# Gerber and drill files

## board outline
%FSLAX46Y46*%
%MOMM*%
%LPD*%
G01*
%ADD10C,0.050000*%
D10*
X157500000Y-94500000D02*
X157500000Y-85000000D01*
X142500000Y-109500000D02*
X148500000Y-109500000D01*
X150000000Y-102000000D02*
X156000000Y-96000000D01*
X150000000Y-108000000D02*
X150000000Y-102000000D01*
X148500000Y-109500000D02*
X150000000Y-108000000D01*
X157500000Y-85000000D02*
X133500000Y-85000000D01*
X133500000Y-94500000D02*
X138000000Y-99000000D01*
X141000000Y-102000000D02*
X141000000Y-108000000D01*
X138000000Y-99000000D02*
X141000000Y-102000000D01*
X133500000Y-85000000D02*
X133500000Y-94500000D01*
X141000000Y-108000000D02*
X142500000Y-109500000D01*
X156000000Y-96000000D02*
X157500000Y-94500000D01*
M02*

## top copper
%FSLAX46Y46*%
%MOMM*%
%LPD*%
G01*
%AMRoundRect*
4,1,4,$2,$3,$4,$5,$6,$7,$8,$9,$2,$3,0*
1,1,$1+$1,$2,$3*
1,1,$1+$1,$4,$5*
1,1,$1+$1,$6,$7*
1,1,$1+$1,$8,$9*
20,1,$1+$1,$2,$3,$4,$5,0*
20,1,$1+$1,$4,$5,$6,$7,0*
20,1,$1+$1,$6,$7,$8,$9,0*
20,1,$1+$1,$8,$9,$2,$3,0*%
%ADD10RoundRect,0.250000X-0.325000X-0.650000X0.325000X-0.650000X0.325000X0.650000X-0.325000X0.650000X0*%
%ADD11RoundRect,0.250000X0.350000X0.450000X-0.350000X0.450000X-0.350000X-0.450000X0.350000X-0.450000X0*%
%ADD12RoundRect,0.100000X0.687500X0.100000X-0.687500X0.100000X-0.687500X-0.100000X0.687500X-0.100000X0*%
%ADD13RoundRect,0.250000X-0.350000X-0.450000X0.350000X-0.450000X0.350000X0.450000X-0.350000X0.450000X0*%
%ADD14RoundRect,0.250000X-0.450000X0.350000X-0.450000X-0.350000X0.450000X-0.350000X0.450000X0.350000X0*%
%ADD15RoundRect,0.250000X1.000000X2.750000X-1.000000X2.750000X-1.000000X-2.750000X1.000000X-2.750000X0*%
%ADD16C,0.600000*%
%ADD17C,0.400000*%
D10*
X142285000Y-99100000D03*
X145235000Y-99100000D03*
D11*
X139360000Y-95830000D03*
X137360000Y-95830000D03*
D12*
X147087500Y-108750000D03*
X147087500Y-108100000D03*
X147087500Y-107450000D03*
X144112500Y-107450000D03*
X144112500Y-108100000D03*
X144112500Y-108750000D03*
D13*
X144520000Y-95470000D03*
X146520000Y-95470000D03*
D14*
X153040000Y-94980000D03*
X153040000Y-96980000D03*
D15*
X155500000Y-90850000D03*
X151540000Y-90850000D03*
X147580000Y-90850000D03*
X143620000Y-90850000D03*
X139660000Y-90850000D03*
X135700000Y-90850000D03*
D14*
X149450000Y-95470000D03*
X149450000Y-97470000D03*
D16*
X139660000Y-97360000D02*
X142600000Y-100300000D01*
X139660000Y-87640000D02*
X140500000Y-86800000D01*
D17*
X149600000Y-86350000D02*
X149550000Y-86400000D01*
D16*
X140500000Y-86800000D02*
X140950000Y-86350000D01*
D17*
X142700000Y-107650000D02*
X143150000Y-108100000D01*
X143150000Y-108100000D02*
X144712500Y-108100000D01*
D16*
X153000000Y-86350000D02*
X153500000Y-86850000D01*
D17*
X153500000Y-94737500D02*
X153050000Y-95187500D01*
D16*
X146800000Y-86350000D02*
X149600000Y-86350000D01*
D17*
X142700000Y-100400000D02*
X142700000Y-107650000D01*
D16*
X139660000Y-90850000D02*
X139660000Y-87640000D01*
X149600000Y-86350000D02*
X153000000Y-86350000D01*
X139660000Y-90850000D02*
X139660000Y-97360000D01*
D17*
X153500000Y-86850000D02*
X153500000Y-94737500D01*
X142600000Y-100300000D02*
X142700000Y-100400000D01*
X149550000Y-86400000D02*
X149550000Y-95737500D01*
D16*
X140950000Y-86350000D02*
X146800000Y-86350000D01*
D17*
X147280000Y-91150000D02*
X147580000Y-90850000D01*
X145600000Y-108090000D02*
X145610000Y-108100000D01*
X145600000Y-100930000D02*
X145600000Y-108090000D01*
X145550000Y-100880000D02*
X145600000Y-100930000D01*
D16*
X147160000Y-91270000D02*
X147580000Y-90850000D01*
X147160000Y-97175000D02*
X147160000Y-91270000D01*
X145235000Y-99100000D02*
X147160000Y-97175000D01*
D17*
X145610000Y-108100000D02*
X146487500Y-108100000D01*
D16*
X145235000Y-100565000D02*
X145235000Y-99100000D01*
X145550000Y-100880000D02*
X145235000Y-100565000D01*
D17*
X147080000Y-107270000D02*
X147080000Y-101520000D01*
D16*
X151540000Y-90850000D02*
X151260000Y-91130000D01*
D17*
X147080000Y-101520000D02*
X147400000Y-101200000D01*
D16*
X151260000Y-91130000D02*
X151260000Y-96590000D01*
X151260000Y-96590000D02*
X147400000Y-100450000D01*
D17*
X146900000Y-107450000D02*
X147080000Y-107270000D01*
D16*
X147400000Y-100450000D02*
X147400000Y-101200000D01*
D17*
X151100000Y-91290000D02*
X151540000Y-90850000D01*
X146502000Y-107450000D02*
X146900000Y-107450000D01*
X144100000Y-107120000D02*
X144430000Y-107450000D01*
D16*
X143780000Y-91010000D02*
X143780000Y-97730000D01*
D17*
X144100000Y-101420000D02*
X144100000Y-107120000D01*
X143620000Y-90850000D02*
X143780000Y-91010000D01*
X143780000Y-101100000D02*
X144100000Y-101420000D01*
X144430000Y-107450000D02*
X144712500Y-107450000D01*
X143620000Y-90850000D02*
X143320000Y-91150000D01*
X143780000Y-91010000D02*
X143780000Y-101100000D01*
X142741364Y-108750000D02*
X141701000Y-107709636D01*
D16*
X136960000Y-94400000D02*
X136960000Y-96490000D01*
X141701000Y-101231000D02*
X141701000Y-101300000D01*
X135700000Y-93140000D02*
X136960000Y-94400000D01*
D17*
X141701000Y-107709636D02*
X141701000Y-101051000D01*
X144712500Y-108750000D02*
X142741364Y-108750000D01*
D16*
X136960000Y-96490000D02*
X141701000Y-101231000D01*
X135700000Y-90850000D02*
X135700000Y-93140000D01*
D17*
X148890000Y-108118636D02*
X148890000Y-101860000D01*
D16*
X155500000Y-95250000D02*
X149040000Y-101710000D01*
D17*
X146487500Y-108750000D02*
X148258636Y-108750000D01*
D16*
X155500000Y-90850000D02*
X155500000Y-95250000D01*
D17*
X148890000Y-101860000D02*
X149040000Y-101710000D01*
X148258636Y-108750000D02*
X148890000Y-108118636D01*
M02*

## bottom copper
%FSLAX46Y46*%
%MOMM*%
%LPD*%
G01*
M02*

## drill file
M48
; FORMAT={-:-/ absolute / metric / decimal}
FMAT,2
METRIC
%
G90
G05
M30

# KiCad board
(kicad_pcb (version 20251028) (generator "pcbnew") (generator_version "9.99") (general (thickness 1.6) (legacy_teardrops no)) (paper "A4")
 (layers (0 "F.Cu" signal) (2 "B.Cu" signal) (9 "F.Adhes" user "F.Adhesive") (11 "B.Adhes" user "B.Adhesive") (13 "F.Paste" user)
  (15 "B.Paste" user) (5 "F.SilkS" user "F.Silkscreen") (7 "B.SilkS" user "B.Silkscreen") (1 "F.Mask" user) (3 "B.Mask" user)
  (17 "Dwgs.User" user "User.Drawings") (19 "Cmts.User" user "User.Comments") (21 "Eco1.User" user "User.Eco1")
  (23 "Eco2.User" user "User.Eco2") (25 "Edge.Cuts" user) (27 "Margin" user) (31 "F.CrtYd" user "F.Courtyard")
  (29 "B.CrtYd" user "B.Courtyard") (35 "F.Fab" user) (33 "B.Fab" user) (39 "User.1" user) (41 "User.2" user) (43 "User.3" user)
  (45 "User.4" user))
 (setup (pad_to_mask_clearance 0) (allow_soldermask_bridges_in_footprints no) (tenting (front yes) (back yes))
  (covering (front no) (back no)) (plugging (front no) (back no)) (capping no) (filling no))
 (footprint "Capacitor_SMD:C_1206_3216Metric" (layer "F.Cu") (at 143.76 99.1)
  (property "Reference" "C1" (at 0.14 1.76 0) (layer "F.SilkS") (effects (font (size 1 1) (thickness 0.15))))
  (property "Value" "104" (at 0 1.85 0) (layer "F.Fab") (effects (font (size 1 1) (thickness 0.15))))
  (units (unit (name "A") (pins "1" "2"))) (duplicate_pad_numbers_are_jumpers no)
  (pad "1" smd roundrect (at -1.475 0) (size 1.15 1.8) (layers "F.Cu" "F.Mask" "F.Paste") (roundrect_rratio 0.217391) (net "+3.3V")
   (tenting (front none) (back none)))
  (pad "2" smd roundrect (at 1.475 0) (size 1.15 1.8) (layers "F.Cu" "F.Mask" "F.Paste") (roundrect_rratio 0.217391) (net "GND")
   (tenting (front none) (back none))))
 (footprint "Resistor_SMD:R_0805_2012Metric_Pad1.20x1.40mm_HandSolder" (layer "F.Cu") (at 138.36 95.83 180)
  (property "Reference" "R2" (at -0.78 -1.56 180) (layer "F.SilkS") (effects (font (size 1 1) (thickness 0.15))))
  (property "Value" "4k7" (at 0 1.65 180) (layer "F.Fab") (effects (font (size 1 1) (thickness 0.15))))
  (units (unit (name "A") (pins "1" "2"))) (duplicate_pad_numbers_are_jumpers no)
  (pad "1" smd roundrect (at -1 0 180) (size 1.2 1.4) (layers "F.Cu" "F.Mask" "F.Paste") (roundrect_rratio 0.208333) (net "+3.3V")
   (tenting (front none) (back none)))
  (pad "2" smd roundrect (at 1 0 180) (size 1.2 1.4) (layers "F.Cu" "F.Mask" "F.Paste") (roundrect_rratio 0.208333) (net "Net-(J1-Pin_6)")
   (tenting (front none) (back none))))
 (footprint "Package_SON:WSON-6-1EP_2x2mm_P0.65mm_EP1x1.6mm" (layer "F.Cu") (at 145.6 108.1 180)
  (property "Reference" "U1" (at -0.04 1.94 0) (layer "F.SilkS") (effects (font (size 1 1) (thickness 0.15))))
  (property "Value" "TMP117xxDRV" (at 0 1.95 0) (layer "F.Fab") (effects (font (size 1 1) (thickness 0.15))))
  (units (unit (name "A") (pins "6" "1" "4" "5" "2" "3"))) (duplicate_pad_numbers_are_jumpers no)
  (pad "1" smd roundrect (at -0.8875 -0.65 180) (size 1.575 0.4) (drill (offset -0.6 0)) (layers "F.Cu" "F.Mask" "F.Paste")
   (roundrect_rratio 0.25) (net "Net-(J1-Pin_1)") (tenting (front none) (back none)))
  (pad "2" smd roundrect (at -0.8875 0 180) (size 1.575 0.4) (drill (offset -0.6 0)) (layers "F.Cu" "F.Mask" "F.Paste")
   (roundrect_rratio 0.25) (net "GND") (tenting (front none) (back none)))
  (pad "3" smd roundrect (at -0.8875 0.65 180) (size 1.575 0.4) (drill (offset -0.6 0)) (layers "F.Cu" "F.Mask" "F.Paste")
   (roundrect_rratio 0.25) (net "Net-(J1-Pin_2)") (tenting (front none) (back none)))
  (pad "4" smd roundrect (at 0.8875 0.65 180) (size 1.575 0.4) (drill (offset 0.6 0)) (layers "F.Cu" "F.Mask" "F.Paste")
   (roundrect_rratio 0.25) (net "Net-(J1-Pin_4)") (tenting (front none) (back none)))
  (pad "5" smd roundrect (at 0.8875 0 180) (size 1.575 0.4) (drill (offset 0.6 0)) (layers "F.Cu" "F.Mask" "F.Paste")
   (roundrect_rratio 0.25) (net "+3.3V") (tenting (front none) (back none)))
  (pad "6" smd roundrect (at 0.8875 -0.65 180) (size 1.575 0.4) (drill (offset 0.6 0)) (layers "F.Cu" "F.Mask" "F.Paste")
   (roundrect_rratio 0.25) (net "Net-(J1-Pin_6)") (tenting (front none) (back none))))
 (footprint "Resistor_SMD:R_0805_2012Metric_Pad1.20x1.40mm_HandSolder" (layer "F.Cu") (at 145.52 95.47)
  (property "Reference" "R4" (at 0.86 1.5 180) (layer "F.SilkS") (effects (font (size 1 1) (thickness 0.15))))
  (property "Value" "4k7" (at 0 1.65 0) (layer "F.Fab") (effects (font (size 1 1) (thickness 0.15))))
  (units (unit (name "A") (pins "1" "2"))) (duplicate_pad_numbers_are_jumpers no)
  (pad "1" smd roundrect (at -1 0) (size 1.2 1.4) (layers "F.Cu" "F.Mask" "F.Paste") (roundrect_rratio 0.208333) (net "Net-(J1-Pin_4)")
   (tenting (front none) (back none)))
  (pad "2" smd roundrect (at 1 0) (size 1.2 1.4) (layers "F.Cu" "F.Mask" "F.Paste") (roundrect_rratio 0.208333) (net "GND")
   (tenting (front none) (back none))))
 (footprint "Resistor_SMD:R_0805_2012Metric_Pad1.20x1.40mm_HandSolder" (layer "F.Cu") (at 153.04 95.98 -90)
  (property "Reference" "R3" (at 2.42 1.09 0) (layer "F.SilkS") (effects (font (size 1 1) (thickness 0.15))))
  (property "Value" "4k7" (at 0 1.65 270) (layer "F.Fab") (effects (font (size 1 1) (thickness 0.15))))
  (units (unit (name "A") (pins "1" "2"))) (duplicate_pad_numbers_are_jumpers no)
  (pad "1" smd roundrect (at -1 0 270) (size 1.2 1.4) (layers "F.Cu" "F.Mask" "F.Paste") (roundrect_rratio 0.208333) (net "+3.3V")
   (tenting (front none) (back none)))
  (pad "2" smd roundrect (at 1 0 270) (size 1.2 1.4) (layers "F.Cu" "F.Mask" "F.Paste") (roundrect_rratio 0.208333) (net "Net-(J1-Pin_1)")
   (tenting (front none) (back none))))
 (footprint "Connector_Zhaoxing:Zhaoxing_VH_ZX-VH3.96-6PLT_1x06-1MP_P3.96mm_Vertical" (layer "F.Cu") (at 145.6 88.85 180)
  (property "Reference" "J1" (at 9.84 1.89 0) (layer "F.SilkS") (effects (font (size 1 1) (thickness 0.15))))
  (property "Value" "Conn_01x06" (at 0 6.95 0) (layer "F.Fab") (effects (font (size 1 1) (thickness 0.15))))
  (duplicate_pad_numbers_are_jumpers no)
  (pad "1" smd roundrect (at -9.9 -2 180) (size 2.5 6) (layers "F.Cu" "F.Mask" "F.Paste") (roundrect_rratio 0.1) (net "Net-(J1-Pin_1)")
   (tenting (front none) (back none)))
  (pad "2" smd roundrect (at -5.94 -2 180) (size 2.5 6) (layers "F.Cu" "F.Mask" "F.Paste") (roundrect_rratio 0.1) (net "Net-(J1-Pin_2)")
   (tenting (front none) (back none)))
  (pad "3" smd roundrect (at -1.98 -2 180) (size 2.5 6) (layers "F.Cu" "F.Mask" "F.Paste") (roundrect_rratio 0.1) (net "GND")
   (tenting (front none) (back none)))
  (pad "4" smd roundrect (at 1.98 -2 180) (size 2.5 6) (layers "F.Cu" "F.Mask" "F.Paste") (roundrect_rratio 0.1) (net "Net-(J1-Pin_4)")
   (tenting (front none) (back none)))
  (pad "5" smd roundrect (at 5.94 -2 180) (size 2.5 6) (layers "F.Cu" "F.Mask" "F.Paste") (roundrect_rratio 0.1) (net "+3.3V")
   (tenting (front none) (back none)))
  (pad "6" smd roundrect (at 9.9 -2 180) (size 2.5 6) (layers "F.Cu" "F.Mask" "F.Paste") (roundrect_rratio 0.1) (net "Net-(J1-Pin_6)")
   (tenting (front none) (back none))))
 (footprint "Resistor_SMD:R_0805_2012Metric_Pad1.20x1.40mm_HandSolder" (layer "F.Cu") (at 149.45 96.47 -90)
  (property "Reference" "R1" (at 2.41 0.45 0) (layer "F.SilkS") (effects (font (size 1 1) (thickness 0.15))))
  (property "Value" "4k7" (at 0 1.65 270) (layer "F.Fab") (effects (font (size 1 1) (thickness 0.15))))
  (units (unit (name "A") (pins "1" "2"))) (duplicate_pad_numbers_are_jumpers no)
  (pad "1" smd roundrect (at -1 0 270) (size 1.2 1.4) (layers "F.Cu" "F.Mask" "F.Paste") (roundrect_rratio 0.208333) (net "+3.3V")
   (tenting (front none) (back none)))
  (pad "2" smd roundrect (at 1 0 270) (size 1.2 1.4) (layers "F.Cu" "F.Mask" "F.Paste") (roundrect_rratio 0.208333) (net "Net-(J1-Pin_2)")
   (tenting (front none) (back none))))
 (gr_line (start 157.5 94.5) (end 157.5 85) (stroke (width 0.05) (type default)) (layer "Edge.Cuts"))
 (gr_line (start 142.5 109.5) (end 148.5 109.5) (stroke (width 0.05) (type default)) (layer "Edge.Cuts"))
 (gr_line (start 150 102) (end 156 96) (stroke (width 0.05) (type default)) (layer "Edge.Cuts"))
 (gr_line (start 150 108) (end 150 102) (stroke (width 0.05) (type default)) (layer "Edge.Cuts"))
 (gr_line (start 148.5 109.5) (end 150 108) (stroke (width 0.05) (type default)) (layer "Edge.Cuts"))
 (gr_line (start 157.5 85) (end 133.5 85) (stroke (width 0.05) (type default)) (layer "Edge.Cuts"))
 (gr_line (start 133.5 94.5) (end 138 99) (stroke (width 0.05) (type default)) (layer "Edge.Cuts"))
 (gr_line (start 141 102) (end 141 108) (stroke (width 0.05) (type default)) (layer "Edge.Cuts"))
 (gr_line (start 138 99) (end 141 102) (stroke (width 0.05) (type default)) (layer "Edge.Cuts"))
 (gr_line (start 133.5 85) (end 133.5 94.5) (stroke (width 0.05) (type default)) (layer "Edge.Cuts"))
 (gr_line (start 141 108) (end 142.5 109.5) (stroke (width 0.05) (type default)) (layer "Edge.Cuts"))
 (gr_line (start 156 96) (end 157.5 94.5) (stroke (width 0.05) (type default)) (layer "Edge.Cuts"))
 (segment (start 139.66 97.36) (end 142.6 100.3) (width 0.6) (layer "F.Cu") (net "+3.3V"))
 (segment (start 139.66 87.64) (end 140.5 86.8) (width 0.6) (layer "F.Cu") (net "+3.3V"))
 (segment (start 149.6 86.35) (end 149.55 86.4) (width 0.4) (layer "F.Cu") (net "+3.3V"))
 (segment (start 140.5 86.8) (end 140.95 86.35) (width 0.6) (layer "F.Cu") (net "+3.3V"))
 (segment (start 142.7 107.65) (end 143.15 108.1) (width 0.4) (layer "F.Cu") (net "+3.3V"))
 (segment (start 143.15 108.1) (end 144.7125 108.1) (width 0.4) (layer "F.Cu") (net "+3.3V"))
 (segment (start 153 86.35) (end 153.5 86.85) (width 0.6) (layer "F.Cu") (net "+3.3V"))
 (segment (start 153.5 94.7375) (end 153.05 95.1875) (width 0.4) (layer "F.Cu") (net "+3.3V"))
 (segment (start 146.8 86.35) (end 149.6 86.35) (width 0.6) (layer "F.Cu") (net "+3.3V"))
 (segment (start 142.7 100.4) (end 142.7 107.65) (width 0.4) (layer "F.Cu") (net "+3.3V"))
 (segment (start 139.66 90.85) (end 139.66 87.64) (width 0.6) (layer "F.Cu") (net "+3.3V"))
 (segment (start 149.6 86.35) (end 153 86.35) (width 0.6) (layer "F.Cu") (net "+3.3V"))
 (segment (start 139.66 90.85) (end 139.66 97.36) (width 0.6) (layer "F.Cu") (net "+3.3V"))
 (segment (start 153.5 86.85) (end 153.5 94.7375) (width 0.4) (layer "F.Cu") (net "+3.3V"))
 (segment (start 142.6 100.3) (end 142.7 100.4) (width 0.4) (layer "F.Cu") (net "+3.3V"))
 (segment (start 149.55 86.4) (end 149.55 95.7375) (width 0.4) (layer "F.Cu") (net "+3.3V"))
 (segment (start 140.95 86.35) (end 146.8 86.35) (width 0.6) (layer "F.Cu") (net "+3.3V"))
 (segment (start 147.28 91.15) (end 147.58 90.85) (width 0.4) (layer "F.Cu") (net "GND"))
 (segment (start 145.6 108.09) (end 145.61 108.1) (width 0.4) (layer "F.Cu") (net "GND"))
 (segment (start 145.6 100.93) (end 145.6 108.09) (width 0.4) (layer "F.Cu") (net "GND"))
 (segment (start 145.55 100.88) (end 145.6 100.93) (width 0.4) (layer "F.Cu") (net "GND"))
 (segment (start 147.16 91.27) (end 147.58 90.85) (width 0.6) (layer "F.Cu") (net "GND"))
 (segment (start 147.16 97.175) (end 147.16 91.27) (width 0.6) (layer "F.Cu") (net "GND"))
 (segment (start 145.235 99.1) (end 147.16 97.175) (width 0.6) (layer "F.Cu") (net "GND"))
 (segment (start 145.61 108.1) (end 146.4875 108.1) (width 0.4) (layer "F.Cu") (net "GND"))
 (segment (start 145.235 100.565) (end 145.235 99.1) (width 0.6) (layer "F.Cu") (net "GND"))
 (segment (start 145.55 100.88) (end 145.235 100.565) (width 0.6) (layer "F.Cu") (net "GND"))
 (segment (start 147.08 107.27) (end 147.08 101.52) (width 0.4) (layer "F.Cu") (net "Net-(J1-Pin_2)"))
 (segment (start 151.54 90.85) (end 151.26 91.13) (width 0.6) (layer "F.Cu") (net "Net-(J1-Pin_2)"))
 (segment (start 147.08 101.52) (end 147.4 101.2) (width 0.4) (layer "F.Cu") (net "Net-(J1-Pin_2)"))
 (segment (start 151.26 91.13) (end 151.26 96.59) (width 0.6) (layer "F.Cu") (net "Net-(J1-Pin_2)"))
 (segment (start 151.26 96.59) (end 147.4 100.45) (width 0.6) (layer "F.Cu") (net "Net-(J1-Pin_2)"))
 (segment (start 146.9 107.45) (end 147.08 107.27) (width 0.4) (layer "F.Cu") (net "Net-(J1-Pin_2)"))
 (segment (start 147.4 100.45) (end 147.4 101.2) (width 0.6) (layer "F.Cu") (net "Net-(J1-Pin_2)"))
 (segment (start 151.1 91.29) (end 151.54 90.85) (width 0.4) (layer "F.Cu") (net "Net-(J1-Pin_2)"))
 (segment (start 146.502 107.45) (end 146.9 107.45) (width 0.4) (layer "F.Cu") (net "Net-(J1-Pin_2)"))
 (segment (start 144.1 107.12) (end 144.43 107.45) (width 0.4) (layer "F.Cu") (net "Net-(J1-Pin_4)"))
 (segment (start 143.78 91.01) (end 143.78 97.73) (width 0.6) (layer "F.Cu") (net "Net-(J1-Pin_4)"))
 (segment (start 144.1 101.42) (end 144.1 107.12) (width 0.4) (layer "F.Cu") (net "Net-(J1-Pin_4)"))
 (segment (start 143.62 90.85) (end 143.78 91.01) (width 0.4) (layer "F.Cu") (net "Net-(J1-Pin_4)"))
 (segment (start 143.78 101.1) (end 144.1 101.42) (width 0.4) (layer "F.Cu") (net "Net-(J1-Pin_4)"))
 (segment (start 144.43 107.45) (end 144.7125 107.45) (width 0.4) (layer "F.Cu") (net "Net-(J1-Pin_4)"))
 (segment (start 143.62 90.85) (end 143.32 91.15) (width 0.4) (layer "F.Cu") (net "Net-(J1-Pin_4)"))
 (segment (start 143.78 91.01) (end 143.78 101.1) (width 0.4) (layer "F.Cu") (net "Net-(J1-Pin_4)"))
 (segment (start 142.741364 108.75) (end 141.701 107.709636) (width 0.4) (layer "F.Cu") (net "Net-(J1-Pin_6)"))
 (segment (start 136.96 94.4) (end 136.96 96.49) (width 0.6) (layer "F.Cu") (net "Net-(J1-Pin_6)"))
 (segment (start 141.701 101.231) (end 141.701 101.3) (width 0.6) (layer "F.Cu") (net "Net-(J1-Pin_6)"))
 (segment (start 135.7 93.14) (end 136.96 94.4) (width 0.6) (layer "F.Cu") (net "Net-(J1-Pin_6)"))
 (segment (start 141.701 107.709636) (end 141.701 101.051) (width 0.4) (layer "F.Cu") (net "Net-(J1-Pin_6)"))
 (segment (start 144.7125 108.75) (end 142.741364 108.75) (width 0.4) (layer "F.Cu") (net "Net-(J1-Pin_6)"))
 (segment (start 136.96 96.49) (end 141.701 101.231) (width 0.6) (layer "F.Cu") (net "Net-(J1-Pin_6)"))
 (segment (start 135.7 90.85) (end 135.7 93.14) (width 0.6) (layer "F.Cu") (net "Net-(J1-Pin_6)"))
 (segment (start 148.89 108.118636) (end 148.89 101.86) (width 0.4) (layer "F.Cu") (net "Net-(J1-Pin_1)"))
 (segment (start 155.5 95.25) (end 149.04 101.71) (width 0.6) (layer "F.Cu") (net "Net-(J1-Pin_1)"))
 (segment (start 146.4875 108.75) (end 148.258636 108.75) (width 0.4) (layer "F.Cu") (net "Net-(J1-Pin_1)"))
 (segment (start 155.5 90.85) (end 155.5 95.25) (width 0.6) (layer "F.Cu") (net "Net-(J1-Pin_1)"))
 (segment (start 148.89 101.86) (end 149.04 101.71) (width 0.4) (layer "F.Cu") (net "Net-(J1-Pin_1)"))
 (segment (start 148.258636 108.75) (end 148.89 108.118636) (width 0.4) (layer "F.Cu") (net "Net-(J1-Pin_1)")))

